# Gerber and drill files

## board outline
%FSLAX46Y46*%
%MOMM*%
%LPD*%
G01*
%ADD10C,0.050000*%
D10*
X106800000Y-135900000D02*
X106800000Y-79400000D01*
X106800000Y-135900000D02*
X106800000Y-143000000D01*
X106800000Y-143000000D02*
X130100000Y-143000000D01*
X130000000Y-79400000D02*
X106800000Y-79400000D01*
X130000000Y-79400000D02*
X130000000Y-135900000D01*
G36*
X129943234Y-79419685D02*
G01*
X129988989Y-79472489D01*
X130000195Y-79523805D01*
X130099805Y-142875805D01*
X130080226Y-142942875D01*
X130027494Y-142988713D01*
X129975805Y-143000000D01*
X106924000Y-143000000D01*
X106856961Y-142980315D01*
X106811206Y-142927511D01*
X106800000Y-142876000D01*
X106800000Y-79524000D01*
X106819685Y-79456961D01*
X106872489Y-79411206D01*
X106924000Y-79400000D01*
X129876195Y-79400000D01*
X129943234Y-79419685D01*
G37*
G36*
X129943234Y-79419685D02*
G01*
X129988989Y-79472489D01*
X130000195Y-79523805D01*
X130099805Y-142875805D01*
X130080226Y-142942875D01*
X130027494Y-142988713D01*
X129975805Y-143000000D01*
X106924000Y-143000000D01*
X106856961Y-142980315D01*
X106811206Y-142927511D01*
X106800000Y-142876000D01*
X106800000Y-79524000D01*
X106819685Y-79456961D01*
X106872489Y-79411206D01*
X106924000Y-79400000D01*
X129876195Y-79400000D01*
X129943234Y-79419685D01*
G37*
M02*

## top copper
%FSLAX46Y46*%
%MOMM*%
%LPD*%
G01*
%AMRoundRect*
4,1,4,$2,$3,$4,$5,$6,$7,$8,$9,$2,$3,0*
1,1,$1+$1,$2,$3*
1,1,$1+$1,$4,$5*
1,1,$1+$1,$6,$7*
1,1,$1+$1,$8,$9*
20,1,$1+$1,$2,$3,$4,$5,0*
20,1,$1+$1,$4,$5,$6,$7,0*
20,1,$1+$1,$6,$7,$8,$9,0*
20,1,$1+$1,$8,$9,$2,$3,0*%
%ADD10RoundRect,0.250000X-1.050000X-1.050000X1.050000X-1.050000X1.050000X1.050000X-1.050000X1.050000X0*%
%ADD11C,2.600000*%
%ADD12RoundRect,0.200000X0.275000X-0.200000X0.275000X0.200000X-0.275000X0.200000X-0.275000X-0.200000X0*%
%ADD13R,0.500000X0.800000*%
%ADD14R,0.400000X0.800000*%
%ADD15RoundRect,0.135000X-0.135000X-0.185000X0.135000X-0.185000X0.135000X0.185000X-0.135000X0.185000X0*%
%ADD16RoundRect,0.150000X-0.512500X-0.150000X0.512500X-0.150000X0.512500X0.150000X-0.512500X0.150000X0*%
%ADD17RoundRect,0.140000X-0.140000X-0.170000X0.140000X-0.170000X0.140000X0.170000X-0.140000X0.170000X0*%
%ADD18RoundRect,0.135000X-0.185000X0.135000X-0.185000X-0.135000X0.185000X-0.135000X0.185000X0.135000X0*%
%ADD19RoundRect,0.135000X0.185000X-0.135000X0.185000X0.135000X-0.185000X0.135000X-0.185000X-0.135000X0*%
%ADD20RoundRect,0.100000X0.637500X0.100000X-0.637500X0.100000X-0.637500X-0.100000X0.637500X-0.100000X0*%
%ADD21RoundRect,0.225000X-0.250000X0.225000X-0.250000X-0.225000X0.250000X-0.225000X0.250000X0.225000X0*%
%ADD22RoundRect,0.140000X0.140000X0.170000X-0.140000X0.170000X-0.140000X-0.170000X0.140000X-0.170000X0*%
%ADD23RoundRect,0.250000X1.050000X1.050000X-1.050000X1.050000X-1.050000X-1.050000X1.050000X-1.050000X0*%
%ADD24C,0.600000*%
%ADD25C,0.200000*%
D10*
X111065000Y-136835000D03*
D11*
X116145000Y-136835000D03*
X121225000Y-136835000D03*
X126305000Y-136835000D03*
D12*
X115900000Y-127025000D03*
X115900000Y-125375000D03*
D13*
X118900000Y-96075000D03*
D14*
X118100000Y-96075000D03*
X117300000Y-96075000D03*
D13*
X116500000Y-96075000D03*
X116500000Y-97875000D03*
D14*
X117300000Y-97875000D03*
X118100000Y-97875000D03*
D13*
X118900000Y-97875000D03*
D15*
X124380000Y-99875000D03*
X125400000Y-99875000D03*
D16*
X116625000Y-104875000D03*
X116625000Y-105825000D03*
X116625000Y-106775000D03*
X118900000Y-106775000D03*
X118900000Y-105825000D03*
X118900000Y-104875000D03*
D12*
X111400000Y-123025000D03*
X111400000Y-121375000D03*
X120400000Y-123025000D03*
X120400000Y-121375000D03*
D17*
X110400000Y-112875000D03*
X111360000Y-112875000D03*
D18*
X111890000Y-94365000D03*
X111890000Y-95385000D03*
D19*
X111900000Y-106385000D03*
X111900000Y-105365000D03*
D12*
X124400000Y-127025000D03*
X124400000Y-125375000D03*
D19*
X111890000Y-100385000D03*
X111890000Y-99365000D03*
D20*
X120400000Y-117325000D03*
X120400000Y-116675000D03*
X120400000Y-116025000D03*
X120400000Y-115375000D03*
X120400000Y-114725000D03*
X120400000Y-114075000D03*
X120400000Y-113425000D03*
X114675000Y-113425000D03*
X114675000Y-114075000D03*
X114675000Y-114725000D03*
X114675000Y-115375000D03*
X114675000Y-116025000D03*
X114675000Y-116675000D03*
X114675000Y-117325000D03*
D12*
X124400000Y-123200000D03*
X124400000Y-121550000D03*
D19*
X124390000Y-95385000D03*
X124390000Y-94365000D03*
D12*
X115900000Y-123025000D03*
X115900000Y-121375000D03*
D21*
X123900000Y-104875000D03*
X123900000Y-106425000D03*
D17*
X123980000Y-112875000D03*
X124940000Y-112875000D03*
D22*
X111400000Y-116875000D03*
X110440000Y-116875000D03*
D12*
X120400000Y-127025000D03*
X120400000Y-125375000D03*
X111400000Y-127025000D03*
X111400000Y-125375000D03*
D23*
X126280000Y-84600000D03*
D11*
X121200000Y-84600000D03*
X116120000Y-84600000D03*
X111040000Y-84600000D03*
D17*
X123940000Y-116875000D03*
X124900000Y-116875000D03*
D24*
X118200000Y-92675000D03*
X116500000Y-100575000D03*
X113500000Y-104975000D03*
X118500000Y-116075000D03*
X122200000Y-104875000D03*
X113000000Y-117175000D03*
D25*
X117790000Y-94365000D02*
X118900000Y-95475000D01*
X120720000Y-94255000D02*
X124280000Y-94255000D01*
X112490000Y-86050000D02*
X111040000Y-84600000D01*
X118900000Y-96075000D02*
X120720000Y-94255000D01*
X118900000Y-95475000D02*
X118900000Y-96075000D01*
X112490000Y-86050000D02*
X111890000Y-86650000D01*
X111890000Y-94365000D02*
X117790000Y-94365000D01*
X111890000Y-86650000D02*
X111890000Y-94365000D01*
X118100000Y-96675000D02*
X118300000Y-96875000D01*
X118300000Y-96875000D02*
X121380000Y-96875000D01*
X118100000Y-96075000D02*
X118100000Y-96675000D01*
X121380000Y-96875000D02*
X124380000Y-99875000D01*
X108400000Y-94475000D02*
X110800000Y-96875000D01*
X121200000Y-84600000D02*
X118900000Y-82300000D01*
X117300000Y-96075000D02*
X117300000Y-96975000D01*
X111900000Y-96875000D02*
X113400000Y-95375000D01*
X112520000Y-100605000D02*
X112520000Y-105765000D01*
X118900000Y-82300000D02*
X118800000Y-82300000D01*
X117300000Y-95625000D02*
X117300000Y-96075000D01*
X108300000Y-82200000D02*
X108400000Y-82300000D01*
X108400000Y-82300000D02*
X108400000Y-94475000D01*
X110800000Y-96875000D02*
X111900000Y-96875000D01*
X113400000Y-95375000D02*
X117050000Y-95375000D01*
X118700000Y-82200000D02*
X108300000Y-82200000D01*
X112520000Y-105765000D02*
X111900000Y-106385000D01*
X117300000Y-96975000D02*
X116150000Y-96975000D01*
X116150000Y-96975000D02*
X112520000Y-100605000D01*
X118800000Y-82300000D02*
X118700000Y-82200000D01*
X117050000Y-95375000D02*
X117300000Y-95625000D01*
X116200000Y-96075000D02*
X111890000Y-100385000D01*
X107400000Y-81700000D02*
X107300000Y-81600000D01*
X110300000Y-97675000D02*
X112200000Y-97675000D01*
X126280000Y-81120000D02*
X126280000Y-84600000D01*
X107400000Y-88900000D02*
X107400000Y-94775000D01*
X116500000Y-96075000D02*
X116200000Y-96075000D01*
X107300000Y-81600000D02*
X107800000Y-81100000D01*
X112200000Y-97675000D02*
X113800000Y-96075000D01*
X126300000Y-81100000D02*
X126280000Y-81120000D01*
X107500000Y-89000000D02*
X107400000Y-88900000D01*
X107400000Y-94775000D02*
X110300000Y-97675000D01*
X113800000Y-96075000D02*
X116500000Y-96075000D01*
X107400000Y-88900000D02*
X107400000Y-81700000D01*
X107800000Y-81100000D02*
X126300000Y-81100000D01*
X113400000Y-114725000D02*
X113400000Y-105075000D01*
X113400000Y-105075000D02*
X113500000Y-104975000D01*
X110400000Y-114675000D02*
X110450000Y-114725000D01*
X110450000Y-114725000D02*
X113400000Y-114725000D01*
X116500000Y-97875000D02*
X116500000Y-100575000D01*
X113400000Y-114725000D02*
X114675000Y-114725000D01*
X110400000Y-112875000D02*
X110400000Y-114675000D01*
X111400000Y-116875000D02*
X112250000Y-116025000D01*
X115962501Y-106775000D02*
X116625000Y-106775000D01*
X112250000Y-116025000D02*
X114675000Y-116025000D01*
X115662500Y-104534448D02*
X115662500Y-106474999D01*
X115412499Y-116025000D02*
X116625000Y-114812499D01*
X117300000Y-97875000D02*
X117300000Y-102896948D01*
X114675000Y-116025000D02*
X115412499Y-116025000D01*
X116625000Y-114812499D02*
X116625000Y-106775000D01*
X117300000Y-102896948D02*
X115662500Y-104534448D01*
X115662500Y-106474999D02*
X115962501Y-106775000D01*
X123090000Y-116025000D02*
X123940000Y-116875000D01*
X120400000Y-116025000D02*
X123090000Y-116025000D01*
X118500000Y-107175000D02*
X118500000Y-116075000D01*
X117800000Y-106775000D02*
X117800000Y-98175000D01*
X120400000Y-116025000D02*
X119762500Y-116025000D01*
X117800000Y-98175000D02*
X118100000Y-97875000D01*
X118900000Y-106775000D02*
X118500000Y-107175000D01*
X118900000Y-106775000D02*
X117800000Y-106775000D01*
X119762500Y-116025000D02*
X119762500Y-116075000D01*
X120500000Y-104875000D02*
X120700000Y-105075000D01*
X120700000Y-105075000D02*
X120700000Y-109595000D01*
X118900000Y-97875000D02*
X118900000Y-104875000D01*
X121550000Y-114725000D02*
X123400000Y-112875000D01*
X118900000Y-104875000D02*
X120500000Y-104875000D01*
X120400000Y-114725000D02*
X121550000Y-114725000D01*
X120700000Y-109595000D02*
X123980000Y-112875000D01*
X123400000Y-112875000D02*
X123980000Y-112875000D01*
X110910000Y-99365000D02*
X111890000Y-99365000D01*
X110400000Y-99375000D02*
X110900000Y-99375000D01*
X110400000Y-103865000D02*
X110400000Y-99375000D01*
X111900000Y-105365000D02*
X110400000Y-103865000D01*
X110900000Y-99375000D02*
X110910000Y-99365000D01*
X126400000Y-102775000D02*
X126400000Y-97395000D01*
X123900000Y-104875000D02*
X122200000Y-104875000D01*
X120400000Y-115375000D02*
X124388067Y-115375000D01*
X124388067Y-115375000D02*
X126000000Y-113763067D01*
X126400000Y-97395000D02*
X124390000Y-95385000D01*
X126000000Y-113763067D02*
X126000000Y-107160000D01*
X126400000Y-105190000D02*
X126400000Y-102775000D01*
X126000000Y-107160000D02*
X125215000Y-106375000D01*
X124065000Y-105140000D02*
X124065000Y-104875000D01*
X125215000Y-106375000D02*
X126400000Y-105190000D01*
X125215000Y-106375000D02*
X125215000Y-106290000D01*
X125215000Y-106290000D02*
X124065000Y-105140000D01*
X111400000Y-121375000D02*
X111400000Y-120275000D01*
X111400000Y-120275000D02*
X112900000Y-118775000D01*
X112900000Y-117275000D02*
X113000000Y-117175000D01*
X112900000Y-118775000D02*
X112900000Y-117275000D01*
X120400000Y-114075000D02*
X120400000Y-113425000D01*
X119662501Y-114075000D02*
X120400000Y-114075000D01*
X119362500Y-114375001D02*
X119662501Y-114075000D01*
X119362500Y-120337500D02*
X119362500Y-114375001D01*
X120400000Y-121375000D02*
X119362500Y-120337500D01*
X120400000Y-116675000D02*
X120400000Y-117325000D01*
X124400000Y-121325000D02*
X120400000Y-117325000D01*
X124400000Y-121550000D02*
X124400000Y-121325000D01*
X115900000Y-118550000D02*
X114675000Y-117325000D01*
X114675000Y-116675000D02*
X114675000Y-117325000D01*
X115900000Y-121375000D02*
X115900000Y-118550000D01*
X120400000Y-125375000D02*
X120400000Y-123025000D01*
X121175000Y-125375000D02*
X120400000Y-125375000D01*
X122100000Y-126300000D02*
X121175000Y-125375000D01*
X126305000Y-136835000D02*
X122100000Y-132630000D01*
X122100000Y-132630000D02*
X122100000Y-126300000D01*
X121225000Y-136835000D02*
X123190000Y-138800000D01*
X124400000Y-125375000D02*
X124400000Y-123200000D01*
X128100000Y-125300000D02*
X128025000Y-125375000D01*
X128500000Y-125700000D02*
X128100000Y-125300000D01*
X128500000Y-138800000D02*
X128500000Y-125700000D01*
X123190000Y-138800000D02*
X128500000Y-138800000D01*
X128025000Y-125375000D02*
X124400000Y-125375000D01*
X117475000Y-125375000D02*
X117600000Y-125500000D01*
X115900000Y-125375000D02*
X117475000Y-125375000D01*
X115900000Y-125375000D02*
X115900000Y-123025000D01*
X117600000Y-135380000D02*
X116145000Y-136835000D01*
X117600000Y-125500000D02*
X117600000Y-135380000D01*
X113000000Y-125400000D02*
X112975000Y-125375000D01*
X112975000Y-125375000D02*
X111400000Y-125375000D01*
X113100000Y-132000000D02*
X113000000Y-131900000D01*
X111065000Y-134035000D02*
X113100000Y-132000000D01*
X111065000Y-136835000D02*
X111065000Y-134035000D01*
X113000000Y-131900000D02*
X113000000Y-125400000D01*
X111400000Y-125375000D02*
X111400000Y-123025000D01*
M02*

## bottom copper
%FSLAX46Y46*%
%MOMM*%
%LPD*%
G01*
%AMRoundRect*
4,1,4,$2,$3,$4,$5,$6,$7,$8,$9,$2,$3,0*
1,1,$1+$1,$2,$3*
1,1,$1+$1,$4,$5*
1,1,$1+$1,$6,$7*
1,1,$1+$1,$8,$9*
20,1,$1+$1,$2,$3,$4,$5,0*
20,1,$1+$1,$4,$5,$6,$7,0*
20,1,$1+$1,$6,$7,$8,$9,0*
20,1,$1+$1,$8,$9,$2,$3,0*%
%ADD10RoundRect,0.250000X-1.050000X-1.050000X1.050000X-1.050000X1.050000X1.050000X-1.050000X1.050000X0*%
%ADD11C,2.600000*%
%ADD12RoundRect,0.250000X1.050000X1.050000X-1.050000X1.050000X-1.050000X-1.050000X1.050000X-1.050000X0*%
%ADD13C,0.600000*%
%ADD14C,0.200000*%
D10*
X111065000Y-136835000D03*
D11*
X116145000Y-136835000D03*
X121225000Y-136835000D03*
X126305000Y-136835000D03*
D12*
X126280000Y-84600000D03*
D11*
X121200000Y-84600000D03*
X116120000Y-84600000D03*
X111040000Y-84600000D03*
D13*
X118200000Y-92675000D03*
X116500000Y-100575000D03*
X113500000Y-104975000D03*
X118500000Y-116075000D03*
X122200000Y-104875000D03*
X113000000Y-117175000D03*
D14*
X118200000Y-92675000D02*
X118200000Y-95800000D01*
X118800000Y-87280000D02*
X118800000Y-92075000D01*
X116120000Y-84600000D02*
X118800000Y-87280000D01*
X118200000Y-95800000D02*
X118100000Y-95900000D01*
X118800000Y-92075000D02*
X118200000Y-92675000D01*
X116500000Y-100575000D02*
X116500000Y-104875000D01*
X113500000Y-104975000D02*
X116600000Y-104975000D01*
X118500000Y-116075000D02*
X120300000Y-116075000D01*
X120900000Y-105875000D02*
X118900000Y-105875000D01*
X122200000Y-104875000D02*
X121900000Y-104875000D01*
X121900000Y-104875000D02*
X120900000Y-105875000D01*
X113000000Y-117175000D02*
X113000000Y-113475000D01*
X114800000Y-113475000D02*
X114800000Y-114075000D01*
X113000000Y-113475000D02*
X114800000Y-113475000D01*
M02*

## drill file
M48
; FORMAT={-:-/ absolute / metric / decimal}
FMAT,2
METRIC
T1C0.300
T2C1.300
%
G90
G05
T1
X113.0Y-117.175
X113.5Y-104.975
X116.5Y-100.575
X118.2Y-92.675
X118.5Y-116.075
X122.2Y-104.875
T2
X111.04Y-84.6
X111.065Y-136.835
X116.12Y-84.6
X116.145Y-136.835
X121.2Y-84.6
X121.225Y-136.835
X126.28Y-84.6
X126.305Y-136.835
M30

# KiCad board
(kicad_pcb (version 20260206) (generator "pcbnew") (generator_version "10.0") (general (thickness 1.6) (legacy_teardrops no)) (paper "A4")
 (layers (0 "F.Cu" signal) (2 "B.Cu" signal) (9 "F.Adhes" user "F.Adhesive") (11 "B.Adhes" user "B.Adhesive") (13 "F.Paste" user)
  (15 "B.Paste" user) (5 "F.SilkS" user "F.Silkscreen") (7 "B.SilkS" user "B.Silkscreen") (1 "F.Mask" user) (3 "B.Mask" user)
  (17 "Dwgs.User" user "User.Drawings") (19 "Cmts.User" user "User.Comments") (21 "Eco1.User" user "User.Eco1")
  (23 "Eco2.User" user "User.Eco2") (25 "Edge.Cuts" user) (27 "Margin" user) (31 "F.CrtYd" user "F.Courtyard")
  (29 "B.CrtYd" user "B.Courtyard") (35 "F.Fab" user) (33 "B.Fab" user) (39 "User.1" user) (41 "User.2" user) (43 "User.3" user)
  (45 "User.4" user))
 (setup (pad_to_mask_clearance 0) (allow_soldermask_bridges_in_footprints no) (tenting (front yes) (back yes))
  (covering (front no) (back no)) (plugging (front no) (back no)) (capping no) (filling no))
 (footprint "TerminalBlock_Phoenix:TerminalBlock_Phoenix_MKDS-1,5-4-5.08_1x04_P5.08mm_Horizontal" (layer "F.Cu") (at 111.065 136.835)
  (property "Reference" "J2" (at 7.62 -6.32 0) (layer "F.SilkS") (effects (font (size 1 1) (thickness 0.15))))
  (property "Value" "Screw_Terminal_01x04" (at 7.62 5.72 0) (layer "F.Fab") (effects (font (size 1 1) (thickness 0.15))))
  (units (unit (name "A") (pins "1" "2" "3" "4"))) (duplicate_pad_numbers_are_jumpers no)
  (pad "1" thru_hole roundrect (at 0 0) (size 2.6 2.6) (drill 1.3) (layers "*.Cu" "*.Mask") (remove_unused_layers no)
   (roundrect_rratio 0.096154) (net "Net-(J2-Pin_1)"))
  (pad "2" thru_hole circle (at 5.08 0) (size 2.6 2.6) (drill 1.3) (layers "*.Cu" "*.Mask") (remove_unused_layers no) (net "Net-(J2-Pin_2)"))
  (pad "3" thru_hole circle (at 10.16 0) (size 2.6 2.6) (drill 1.3) (layers "*.Cu" "*.Mask") (remove_unused_layers no)
   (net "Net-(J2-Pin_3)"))
  (pad "4" thru_hole circle (at 15.24 0) (size 2.6 2.6) (drill 1.3) (layers "*.Cu" "*.Mask") (remove_unused_layers no)
   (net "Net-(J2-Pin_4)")))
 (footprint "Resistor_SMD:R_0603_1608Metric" (layer "F.Cu") (at 115.9 126.2 90)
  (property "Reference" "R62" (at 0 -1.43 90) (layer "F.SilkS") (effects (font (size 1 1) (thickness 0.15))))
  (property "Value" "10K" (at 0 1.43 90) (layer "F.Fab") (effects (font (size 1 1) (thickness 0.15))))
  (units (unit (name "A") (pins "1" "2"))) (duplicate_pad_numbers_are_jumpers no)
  (pad "1" smd roundrect (at -0.825 0 90) (size 0.8 0.95) (layers "F.Cu" "F.Mask" "F.Paste") (roundrect_rratio 0.25) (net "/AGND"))
  (pad "2" smd roundrect (at 0.825 0 90) (size 0.8 0.95) (layers "F.Cu" "F.Mask" "F.Paste") (roundrect_rratio 0.25) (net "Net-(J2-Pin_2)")))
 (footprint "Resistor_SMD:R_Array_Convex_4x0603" (layer "F.Cu") (at 117.7 96.975 -90)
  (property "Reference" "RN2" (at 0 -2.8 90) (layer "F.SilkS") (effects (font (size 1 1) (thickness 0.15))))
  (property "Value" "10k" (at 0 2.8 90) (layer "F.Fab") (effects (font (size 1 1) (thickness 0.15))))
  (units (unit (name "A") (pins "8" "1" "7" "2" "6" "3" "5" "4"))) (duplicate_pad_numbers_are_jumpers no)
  (pad "1" smd rect (at -0.9 -1.2 270) (size 0.8 0.5) (layers "F.Cu" "F.Mask" "F.Paste") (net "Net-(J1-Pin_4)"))
  (pad "2" smd rect (at -0.9 -0.4 270) (size 0.8 0.4) (layers "F.Cu" "F.Mask" "F.Paste") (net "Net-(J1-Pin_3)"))
  (pad "3" smd rect (at -0.9 0.4 270) (size 0.8 0.4) (layers "F.Cu" "F.Mask" "F.Paste") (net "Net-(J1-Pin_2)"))
  (pad "4" smd rect (at -0.9 1.2 270) (size 0.8 0.5) (layers "F.Cu" "F.Mask" "F.Paste") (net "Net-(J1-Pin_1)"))
  (pad "5" smd rect (at 0.9 1.2 270) (size 0.8 0.5) (layers "F.Cu" "F.Mask" "F.Paste") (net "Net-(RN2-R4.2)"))
  (pad "6" smd rect (at 0.9 0.4 270) (size 0.8 0.4) (layers "F.Cu" "F.Mask" "F.Paste") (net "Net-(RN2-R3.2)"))
  (pad "7" smd rect (at 0.9 -0.4 270) (size 0.8 0.4) (layers "F.Cu" "B.Mask" "F.Paste") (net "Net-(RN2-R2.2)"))
  (pad "8" smd rect (at 0.9 -1.2 270) (size 0.8 0.5) (layers "F.Cu" "F.Mask" "F.Paste") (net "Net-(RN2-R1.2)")))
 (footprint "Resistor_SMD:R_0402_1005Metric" (layer "F.Cu") (at 124.89 99.875)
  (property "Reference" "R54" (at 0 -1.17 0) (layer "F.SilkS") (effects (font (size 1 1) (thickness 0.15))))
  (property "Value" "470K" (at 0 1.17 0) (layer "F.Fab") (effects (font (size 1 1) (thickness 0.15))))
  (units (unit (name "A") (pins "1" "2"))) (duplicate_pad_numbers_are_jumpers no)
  (pad "1" smd roundrect (at -0.51 0) (size 0.54 0.64) (layers "F.Cu" "F.Mask" "F.Paste") (roundrect_rratio 0.25) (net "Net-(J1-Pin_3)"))
  (pad "2" smd roundrect (at 0.51 0) (size 0.54 0.64) (layers "F.Cu" "F.Mask" "F.Paste") (roundrect_rratio 0.25) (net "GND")))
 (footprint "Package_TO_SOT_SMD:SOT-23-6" (layer "F.Cu") (at 117.7625 105.825)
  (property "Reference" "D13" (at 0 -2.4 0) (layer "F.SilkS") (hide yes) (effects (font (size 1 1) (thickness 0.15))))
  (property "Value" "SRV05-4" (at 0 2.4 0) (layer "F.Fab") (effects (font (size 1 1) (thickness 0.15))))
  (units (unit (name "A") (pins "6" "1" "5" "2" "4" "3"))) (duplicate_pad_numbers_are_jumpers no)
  (pad "1" smd roundrect (at -1.1375 -0.95) (size 1.325 0.6) (layers "F.Cu" "F.Mask" "F.Paste") (roundrect_rratio 0.25)
   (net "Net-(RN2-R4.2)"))
  (pad "2" smd roundrect (at -1.1375 0) (size 1.325 0.6) (layers "F.Cu" "F.Mask" "F.Paste") (roundrect_rratio 0.25) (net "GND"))
  (pad "3" smd roundrect (at -1.1375 0.95) (size 1.325 0.6) (layers "F.Cu" "F.Mask" "F.Paste") (roundrect_rratio 0.25)
   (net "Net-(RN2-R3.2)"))
  (pad "4" smd roundrect (at 1.1375 0.95) (size 1.325 0.6) (layers "F.Cu" "F.Mask" "F.Paste") (roundrect_rratio 0.25) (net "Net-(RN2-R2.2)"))
  (pad "5" smd roundrect (at 1.1375 0) (size 1.325 0.6) (layers "F.Cu" "F.Mask" "F.Paste") (roundrect_rratio 0.25) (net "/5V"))
  (pad "6" smd roundrect (at 1.1375 -0.95) (size 1.325 0.6) (layers "F.Cu" "F.Mask" "F.Paste") (roundrect_rratio 0.25)
   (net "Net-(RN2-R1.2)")))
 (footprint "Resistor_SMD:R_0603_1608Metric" (layer "F.Cu") (at 111.4 122.2 90)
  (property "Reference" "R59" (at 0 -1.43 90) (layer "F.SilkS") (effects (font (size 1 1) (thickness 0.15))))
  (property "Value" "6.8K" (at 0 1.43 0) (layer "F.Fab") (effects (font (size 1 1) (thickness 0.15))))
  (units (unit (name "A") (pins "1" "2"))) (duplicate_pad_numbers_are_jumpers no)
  (pad "1" smd roundrect (at -0.825 0 90) (size 0.8 0.95) (layers "F.Cu" "F.Mask" "F.Paste") (roundrect_rratio 0.25) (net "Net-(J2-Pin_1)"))
  (pad "2" smd roundrect (at 0.825 0 90) (size 0.8 0.95) (layers "F.Cu" "F.Mask" "F.Paste") (roundrect_rratio 0.25) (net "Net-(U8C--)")))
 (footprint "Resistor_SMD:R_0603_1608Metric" (layer "F.Cu") (at 120.4 122.2 90)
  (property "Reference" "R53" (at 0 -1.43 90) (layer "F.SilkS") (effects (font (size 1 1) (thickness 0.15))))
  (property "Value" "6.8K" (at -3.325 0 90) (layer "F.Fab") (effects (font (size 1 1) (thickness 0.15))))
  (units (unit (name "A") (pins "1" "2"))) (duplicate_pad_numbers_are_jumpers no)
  (pad "1" smd roundrect (at -0.825 0 90) (size 0.8 0.95) (layers "F.Cu" "F.Mask" "F.Paste") (roundrect_rratio 0.25) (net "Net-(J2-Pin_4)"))
  (pad "2" smd roundrect (at 0.825 0 90) (size 0.8 0.95) (layers "F.Cu" "F.Mask" "F.Paste") (roundrect_rratio 0.25) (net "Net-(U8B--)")))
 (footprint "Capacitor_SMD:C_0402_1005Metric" (layer "F.Cu") (at 110.88 112.875)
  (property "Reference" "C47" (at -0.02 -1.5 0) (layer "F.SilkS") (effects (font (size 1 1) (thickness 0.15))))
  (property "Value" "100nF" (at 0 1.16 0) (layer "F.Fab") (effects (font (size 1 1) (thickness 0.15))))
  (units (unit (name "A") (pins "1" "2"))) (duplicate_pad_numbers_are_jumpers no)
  (pad "1" smd roundrect (at -0.48 0) (size 0.56 0.62) (layers "F.Cu" "F.Mask" "F.Paste") (roundrect_rratio 0.25) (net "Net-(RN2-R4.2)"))
  (pad "2" smd roundrect (at 0.48 0) (size 0.56 0.62) (layers "F.Cu" "F.Mask" "F.Paste") (roundrect_rratio 0.25) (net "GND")))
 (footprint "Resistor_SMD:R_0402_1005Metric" (layer "F.Cu") (at 111.89 94.875 -90)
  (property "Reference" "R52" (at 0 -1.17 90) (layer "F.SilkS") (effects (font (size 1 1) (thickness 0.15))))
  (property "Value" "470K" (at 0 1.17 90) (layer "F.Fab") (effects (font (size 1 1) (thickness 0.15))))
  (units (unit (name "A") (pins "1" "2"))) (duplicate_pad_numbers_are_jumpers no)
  (pad "1" smd roundrect (at -0.51 0 270) (size 0.54 0.64) (layers "F.Cu" "F.Mask" "F.Paste") (roundrect_rratio 0.25) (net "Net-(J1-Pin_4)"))
  (pad "2" smd roundrect (at 0.51 0 270) (size 0.54 0.64) (layers "F.Cu" "F.Mask" "F.Paste") (roundrect_rratio 0.25) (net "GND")))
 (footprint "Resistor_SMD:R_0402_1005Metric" (layer "F.Cu") (at 111.9 105.875 90)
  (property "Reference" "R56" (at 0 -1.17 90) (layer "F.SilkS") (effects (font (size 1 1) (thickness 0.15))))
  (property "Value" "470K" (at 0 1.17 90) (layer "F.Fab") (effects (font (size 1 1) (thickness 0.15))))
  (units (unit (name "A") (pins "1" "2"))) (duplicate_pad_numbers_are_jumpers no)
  (pad "1" smd roundrect (at -0.51 0 90) (size 0.54 0.64) (layers "F.Cu" "F.Mask" "F.Paste") (roundrect_rratio 0.25) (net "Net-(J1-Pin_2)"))
  (pad "2" smd roundrect (at 0.51 0 90) (size 0.54 0.64) (layers "F.Cu" "F.Mask" "F.Paste") (roundrect_rratio 0.25) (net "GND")))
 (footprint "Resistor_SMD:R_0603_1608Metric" (layer "F.Cu") (at 124.4 126.2 90)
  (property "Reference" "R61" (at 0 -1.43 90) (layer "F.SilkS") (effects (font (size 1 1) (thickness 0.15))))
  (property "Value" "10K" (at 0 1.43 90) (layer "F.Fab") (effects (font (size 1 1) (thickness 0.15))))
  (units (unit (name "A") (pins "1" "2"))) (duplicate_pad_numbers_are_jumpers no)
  (pad "1" smd roundrect (at -0.825 0 90) (size 0.8 0.95) (layers "F.Cu" "F.Mask" "F.Paste") (roundrect_rratio 0.25) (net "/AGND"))
  (pad "2" smd roundrect (at 0.825 0 90) (size 0.8 0.95) (layers "F.Cu" "F.Mask" "F.Paste") (roundrect_rratio 0.25) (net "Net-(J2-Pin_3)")))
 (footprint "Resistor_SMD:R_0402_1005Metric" (layer "F.Cu") (at 111.89 99.875 90)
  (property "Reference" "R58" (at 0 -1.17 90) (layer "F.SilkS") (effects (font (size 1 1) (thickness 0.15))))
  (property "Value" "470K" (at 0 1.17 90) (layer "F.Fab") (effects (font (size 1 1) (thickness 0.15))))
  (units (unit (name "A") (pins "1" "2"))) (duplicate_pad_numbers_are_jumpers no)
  (pad "1" smd roundrect (at -0.51 0 90) (size 0.54 0.64) (layers "F.Cu" "F.Mask" "F.Paste") (roundrect_rratio 0.25) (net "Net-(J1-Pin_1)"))
  (pad "2" smd roundrect (at 0.51 0 90) (size 0.54 0.64) (layers "F.Cu" "F.Mask" "F.Paste") (roundrect_rratio 0.25) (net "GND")))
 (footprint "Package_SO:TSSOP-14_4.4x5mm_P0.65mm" (layer "F.Cu") (at 117.5375 115.375 180)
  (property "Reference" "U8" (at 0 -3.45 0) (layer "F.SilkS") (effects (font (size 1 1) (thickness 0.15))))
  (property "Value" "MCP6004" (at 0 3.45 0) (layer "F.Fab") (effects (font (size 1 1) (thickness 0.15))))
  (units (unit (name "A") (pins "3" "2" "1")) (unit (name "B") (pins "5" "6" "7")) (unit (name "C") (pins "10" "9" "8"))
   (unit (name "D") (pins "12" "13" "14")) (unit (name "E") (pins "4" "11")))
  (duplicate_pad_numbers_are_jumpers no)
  (pad "1" smd roundrect (at -2.8625 -1.95 180) (size 1.475 0.4) (layers "F.Cu" "F.Mask" "F.Paste") (roundrect_rratio 0.25)
   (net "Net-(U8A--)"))
  (pad "2" smd roundrect (at -2.8625 -1.3 180) (size 1.475 0.4) (layers "F.Cu" "F.Mask" "F.Paste") (roundrect_rratio 0.25)
   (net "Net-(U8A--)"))
  (pad "3" smd roundrect (at -2.8625 -0.65 180) (size 1.475 0.4) (layers "F.Cu" "F.Mask" "F.Paste") (roundrect_rratio 0.25)
   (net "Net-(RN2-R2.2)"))
  (pad "4" smd roundrect (at -2.8625 0 180) (size 1.475 0.4) (layers "F.Cu" "F.Mask" "F.Paste") (roundrect_rratio 0.25) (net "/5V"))
  (pad "5" smd roundrect (at -2.8625 0.65 180) (size 1.475 0.4) (layers "F.Cu" "F.Mask" "F.Paste") (roundrect_rratio 0.25)
   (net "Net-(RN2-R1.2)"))
  (pad "6" smd roundrect (at -2.8625 1.3 180) (size 1.475 0.4) (layers "F.Cu" "F.Mask" "F.Paste") (roundrect_rratio 0.25)
   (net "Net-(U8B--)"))
  (pad "7" smd roundrect (at -2.8625 1.95 180) (size 1.475 0.4) (layers "F.Cu" "F.Mask" "F.Paste") (roundrect_rratio 0.25)
   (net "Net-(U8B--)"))
  (pad "8" smd roundrect (at 2.8625 1.95 180) (size 1.475 0.4) (layers "F.Cu" "F.Mask" "F.Paste") (roundrect_rratio 0.25)
   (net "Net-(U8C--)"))
  (pad "9" smd roundrect (at 2.8625 1.3 180) (size 1.475 0.4) (layers "F.Cu" "F.Mask" "F.Paste") (roundrect_rratio 0.25) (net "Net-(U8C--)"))
  (pad "10" smd roundrect (at 2.8625 0.65 180) (size 1.475 0.4) (layers "F.Cu" "F.Mask" "F.Paste") (roundrect_rratio 0.25)
   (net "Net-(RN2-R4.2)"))
  (pad "11" smd roundrect (at 2.8625 0 180) (size 1.475 0.4) (layers "F.Cu" "F.Mask" "F.Paste") (roundrect_rratio 0.25)
   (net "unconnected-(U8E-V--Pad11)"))
  (pad "12" smd roundrect (at 2.8625 -0.65 180) (size 1.475 0.4) (layers "F.Cu" "F.Mask" "F.Paste") (roundrect_rratio 0.25)
   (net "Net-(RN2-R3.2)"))
  (pad "13" smd roundrect (at 2.8625 -1.3 180) (size 1.475 0.4) (layers "F.Cu" "F.Mask" "F.Paste") (roundrect_rratio 0.25)
   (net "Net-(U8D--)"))
  (pad "14" smd roundrect (at 2.8625 -1.95 180) (size 1.475 0.4) (layers "F.Cu" "F.Mask" "F.Paste") (roundrect_rratio 0.25)
   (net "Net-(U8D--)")))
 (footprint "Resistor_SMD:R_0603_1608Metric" (layer "F.Cu") (at 124.4 122.375 90)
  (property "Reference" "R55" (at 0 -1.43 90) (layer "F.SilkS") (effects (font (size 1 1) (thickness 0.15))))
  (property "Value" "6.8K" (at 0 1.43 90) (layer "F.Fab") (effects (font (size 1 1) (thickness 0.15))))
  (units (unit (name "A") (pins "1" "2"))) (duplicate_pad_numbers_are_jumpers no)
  (pad "1" smd roundrect (at -0.825 0 90) (size 0.8 0.95) (layers "F.Cu" "F.Mask" "F.Paste") (roundrect_rratio 0.25) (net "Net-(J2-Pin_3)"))
  (pad "2" smd roundrect (at 0.825 0 90) (size 0.8 0.95) (layers "F.Cu" "F.Mask" "F.Paste") (roundrect_rratio 0.25) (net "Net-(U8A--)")))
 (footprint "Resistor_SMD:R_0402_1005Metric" (layer "F.Cu") (at 124.39 94.875 90)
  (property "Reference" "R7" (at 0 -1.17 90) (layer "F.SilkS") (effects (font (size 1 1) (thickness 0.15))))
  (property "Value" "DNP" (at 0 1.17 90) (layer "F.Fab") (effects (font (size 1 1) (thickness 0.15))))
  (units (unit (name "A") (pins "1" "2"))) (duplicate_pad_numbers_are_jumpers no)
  (pad "1" smd roundrect (at -0.51 0 90) (size 0.54 0.64) (layers "F.Cu" "F.Mask" "F.Paste") (roundrect_rratio 0.25) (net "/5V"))
  (pad "2" smd roundrect (at 0.51 0 90) (size 0.54 0.64) (layers "F.Cu" "F.Mask" "F.Paste") (roundrect_rratio 0.25) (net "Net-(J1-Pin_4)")))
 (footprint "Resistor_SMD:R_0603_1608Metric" (layer "F.Cu") (at 115.9 122.2 90)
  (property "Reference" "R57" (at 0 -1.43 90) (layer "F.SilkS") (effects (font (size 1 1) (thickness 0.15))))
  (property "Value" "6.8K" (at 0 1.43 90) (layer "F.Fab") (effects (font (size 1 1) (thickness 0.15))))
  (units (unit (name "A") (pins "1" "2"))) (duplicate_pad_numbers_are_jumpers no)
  (pad "1" smd roundrect (at -0.825 0 90) (size 0.8 0.95) (layers "F.Cu" "F.Mask" "F.Paste") (roundrect_rratio 0.25) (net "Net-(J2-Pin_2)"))
  (pad "2" smd roundrect (at 0.825 0 90) (size 0.8 0.95) (layers "F.Cu" "F.Mask" "F.Paste") (roundrect_rratio 0.25) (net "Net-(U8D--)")))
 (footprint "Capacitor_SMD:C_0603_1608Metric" (layer "F.Cu") (at 123.9 105.65 -90)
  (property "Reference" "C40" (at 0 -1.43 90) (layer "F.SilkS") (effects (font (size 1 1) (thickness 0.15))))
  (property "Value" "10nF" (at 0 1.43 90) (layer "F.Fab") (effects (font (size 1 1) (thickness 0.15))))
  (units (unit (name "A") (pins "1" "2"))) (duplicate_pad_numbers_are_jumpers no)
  (pad "1" smd roundrect (at -0.775 0 270) (size 0.9 0.95) (layers "F.Cu" "F.Mask" "F.Paste") (roundrect_rratio 0.25) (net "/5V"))
  (pad "2" smd roundrect (at 0.775 0 270) (size 0.9 0.95) (layers "F.Cu" "F.Mask" "F.Paste") (roundrect_rratio 0.25) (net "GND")))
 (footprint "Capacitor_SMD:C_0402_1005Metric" (layer "F.Cu") (at 124.46 112.875)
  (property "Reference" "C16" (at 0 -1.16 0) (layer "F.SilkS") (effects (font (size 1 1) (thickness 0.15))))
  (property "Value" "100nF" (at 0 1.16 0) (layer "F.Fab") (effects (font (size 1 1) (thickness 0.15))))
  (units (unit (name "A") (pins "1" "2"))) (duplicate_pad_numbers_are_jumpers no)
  (pad "1" smd roundrect (at -0.48 0) (size 0.56 0.62) (layers "F.Cu" "F.Mask" "F.Paste") (roundrect_rratio 0.25) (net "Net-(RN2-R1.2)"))
  (pad "2" smd roundrect (at 0.48 0) (size 0.56 0.62) (layers "F.Cu" "F.Mask" "F.Paste") (roundrect_rratio 0.25) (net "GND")))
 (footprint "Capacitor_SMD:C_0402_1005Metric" (layer "F.Cu") (at 110.92 116.875 180)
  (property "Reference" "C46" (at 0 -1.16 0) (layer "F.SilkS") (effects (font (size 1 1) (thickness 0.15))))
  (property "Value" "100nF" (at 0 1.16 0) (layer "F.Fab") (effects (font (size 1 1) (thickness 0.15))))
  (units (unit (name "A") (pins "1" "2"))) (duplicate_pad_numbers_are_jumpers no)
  (pad "1" smd roundrect (at -0.48 0 180) (size 0.56 0.62) (layers "F.Cu" "F.Mask" "F.Paste") (roundrect_rratio 0.25) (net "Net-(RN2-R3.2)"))
  (pad "2" smd roundrect (at 0.48 0 180) (size 0.56 0.62) (layers "F.Cu" "F.Mask" "F.Paste") (roundrect_rratio 0.25) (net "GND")))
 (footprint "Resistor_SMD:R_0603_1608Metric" (layer "F.Cu") (at 120.4 126.2 90)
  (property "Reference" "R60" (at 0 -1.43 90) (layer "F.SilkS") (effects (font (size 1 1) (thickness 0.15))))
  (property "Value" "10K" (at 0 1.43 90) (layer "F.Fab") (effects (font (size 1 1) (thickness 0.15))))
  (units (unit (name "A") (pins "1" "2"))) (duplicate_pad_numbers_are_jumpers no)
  (pad "1" smd roundrect (at -0.825 0 90) (size 0.8 0.95) (layers "F.Cu" "F.Mask" "F.Paste") (roundrect_rratio 0.25) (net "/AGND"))
  (pad "2" smd roundrect (at 0.825 0 90) (size 0.8 0.95) (layers "F.Cu" "F.Mask" "F.Paste") (roundrect_rratio 0.25) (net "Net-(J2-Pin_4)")))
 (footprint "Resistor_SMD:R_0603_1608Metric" (layer "F.Cu") (at 111.4 126.2 90)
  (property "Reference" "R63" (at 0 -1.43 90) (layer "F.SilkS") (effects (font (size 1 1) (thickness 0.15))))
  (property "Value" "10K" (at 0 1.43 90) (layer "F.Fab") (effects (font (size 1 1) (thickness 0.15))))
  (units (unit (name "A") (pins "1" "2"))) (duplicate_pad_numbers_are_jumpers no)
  (pad "1" smd roundrect (at -0.825 0 90) (size 0.8 0.95) (layers "F.Cu" "F.Mask" "F.Paste") (roundrect_rratio 0.25) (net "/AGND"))
  (pad "2" smd roundrect (at 0.825 0 90) (size 0.8 0.95) (layers "F.Cu" "F.Mask" "F.Paste") (roundrect_rratio 0.25) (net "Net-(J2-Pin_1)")))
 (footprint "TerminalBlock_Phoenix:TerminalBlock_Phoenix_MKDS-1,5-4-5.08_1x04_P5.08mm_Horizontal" (layer "F.Cu") (at 126.28 84.6 180)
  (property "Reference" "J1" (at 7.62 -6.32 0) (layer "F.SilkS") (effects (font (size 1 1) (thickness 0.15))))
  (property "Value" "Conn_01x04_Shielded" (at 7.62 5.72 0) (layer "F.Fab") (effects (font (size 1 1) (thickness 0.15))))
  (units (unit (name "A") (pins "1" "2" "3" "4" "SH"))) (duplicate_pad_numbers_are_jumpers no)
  (pad "1" thru_hole roundrect (at 0 0 180) (size 2.6 2.6) (drill 1.3) (layers "*.Cu" "*.Mask") (remove_unused_layers no)
   (roundrect_rratio 0.096154) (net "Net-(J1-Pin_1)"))
  (pad "2" thru_hole circle (at 5.08 0 180) (size 2.6 2.6) (drill 1.3) (layers "*.Cu" "*.Mask") (remove_unused_layers no)
   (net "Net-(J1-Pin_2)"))
  (pad "3" thru_hole circle (at 10.16 0 180) (size 2.6 2.6) (drill 1.3) (layers "*.Cu" "*.Mask") (remove_unused_layers no)
   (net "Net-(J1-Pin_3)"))
  (pad "4" thru_hole circle (at 15.24 0 180) (size 2.6 2.6) (drill 1.3) (layers "*.Cu" "*.Mask") (remove_unused_layers no)
   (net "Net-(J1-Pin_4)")))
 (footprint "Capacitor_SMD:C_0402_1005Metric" (layer "F.Cu") (at 124.42 116.875)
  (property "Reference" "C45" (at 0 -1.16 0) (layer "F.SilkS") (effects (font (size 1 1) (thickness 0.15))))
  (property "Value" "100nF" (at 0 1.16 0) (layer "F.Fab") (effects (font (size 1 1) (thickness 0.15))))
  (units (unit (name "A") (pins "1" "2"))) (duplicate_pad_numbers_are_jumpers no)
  (pad "1" smd roundrect (at -0.48 0) (size 0.56 0.62) (layers "F.Cu" "F.Mask" "F.Paste") (roundrect_rratio 0.25) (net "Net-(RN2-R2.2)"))
  (pad "2" smd roundrect (at 0.48 0) (size 0.56 0.62) (layers "F.Cu" "F.Mask" "F.Paste") (roundrect_rratio 0.25) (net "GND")))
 (gr_line (start 106.8 135.9) (end 106.8 79.4) (stroke (width 0.05) (type default)) (layer "Edge.Cuts"))
 (gr_line (start 106.8 135.9) (end 106.8 143) (stroke (width 0.05) (type default)) (layer "Edge.Cuts"))
 (gr_line (start 106.8 143) (end 130.1 143) (stroke (width 0.05) (type default)) (layer "Edge.Cuts"))
 (gr_line (start 130 79.4) (end 106.8 79.4) (stroke (width 0.05) (type default)) (layer "Edge.Cuts"))
 (gr_line (start 130 79.4) (end 130 135.9) (stroke (width 0.05) (type default)) (layer "Edge.Cuts"))
 (segment (start 117.79 94.365) (end 118.9 95.475) (width 0.2) (layer "F.Cu") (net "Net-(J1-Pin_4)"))
 (segment (start 120.72 94.255) (end 124.28 94.255) (width 0.2) (layer "F.Cu") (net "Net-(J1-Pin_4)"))
 (segment (start 112.49 86.05) (end 111.04 84.6) (width 0.2) (layer "F.Cu") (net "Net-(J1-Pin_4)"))
 (segment (start 118.9 96.075) (end 120.72 94.255) (width 0.2) (layer "F.Cu") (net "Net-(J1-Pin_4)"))
 (segment (start 118.9 95.475) (end 118.9 96.075) (width 0.2) (layer "F.Cu") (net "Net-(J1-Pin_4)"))
 (segment (start 112.49 86.05) (end 111.89 86.65) (width 0.2) (layer "F.Cu") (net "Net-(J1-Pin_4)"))
 (segment (start 111.89 94.365) (end 117.79 94.365) (width 0.2) (layer "F.Cu") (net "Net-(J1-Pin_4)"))
 (segment (start 111.89 86.65) (end 111.89 94.365) (width 0.2) (layer "F.Cu") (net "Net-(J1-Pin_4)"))
 (segment (start 118.1 96.675) (end 118.3 96.875) (width 0.2) (layer "F.Cu") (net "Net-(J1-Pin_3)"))
 (segment (start 118.3 96.875) (end 121.38 96.875) (width 0.2) (layer "F.Cu") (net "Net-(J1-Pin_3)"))
 (segment (start 118.1 96.075) (end 118.1 96.675) (width 0.2) (layer "F.Cu") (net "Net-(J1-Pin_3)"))
 (segment (start 121.38 96.875) (end 124.38 99.875) (width 0.2) (layer "F.Cu") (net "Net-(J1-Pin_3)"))
 (via (at 118.2 92.675) (size 0.6) (drill 0.3) (layers "F.Cu" "B.Cu") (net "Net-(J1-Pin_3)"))
 (segment (start 118.2 92.675) (end 118.2 95.8) (width 0.2) (layer "B.Cu") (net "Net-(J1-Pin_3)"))
 (segment (start 118.8 87.28) (end 118.8 92.075) (width 0.2) (layer "B.Cu") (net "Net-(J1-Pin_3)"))
 (segment (start 116.12 84.6) (end 118.8 87.28) (width 0.2) (layer "B.Cu") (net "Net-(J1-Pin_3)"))
 (segment (start 118.2 95.8) (end 118.1 95.9) (width 0.2) (layer "B.Cu") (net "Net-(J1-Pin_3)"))
 (segment (start 118.8 92.075) (end 118.2 92.675) (width 0.2) (layer "B.Cu") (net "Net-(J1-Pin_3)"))
 (segment (start 108.4 94.475) (end 110.8 96.875) (width 0.2) (layer "F.Cu") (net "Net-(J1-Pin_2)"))
 (segment (start 121.2 84.6) (end 118.9 82.3) (width 0.2) (layer "F.Cu") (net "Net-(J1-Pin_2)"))
 (segment (start 117.3 96.075) (end 117.3 96.975) (width 0.2) (layer "F.Cu") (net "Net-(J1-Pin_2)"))
 (segment (start 111.9 96.875) (end 113.4 95.375) (width 0.2) (layer "F.Cu") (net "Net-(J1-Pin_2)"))
 (segment (start 112.52 100.605) (end 112.52 105.765) (width 0.2) (layer "F.Cu") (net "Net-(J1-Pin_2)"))
 (segment (start 118.9 82.3) (end 118.8 82.3) (width 0.2) (layer "F.Cu") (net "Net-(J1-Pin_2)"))
 (segment (start 117.3 95.625) (end 117.3 96.075) (width 0.2) (layer "F.Cu") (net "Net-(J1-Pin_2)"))
 (segment (start 108.3 82.2) (end 108.4 82.3) (width 0.2) (layer "F.Cu") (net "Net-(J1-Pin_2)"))
 (segment (start 108.4 82.3) (end 108.4 94.475) (width 0.2) (layer "F.Cu") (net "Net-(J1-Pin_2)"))
 (segment (start 110.8 96.875) (end 111.9 96.875) (width 0.2) (layer "F.Cu") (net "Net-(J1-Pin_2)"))
 (segment (start 113.4 95.375) (end 117.05 95.375) (width 0.2) (layer "F.Cu") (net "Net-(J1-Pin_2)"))
 (segment (start 118.7 82.2) (end 108.3 82.2) (width 0.2) (layer "F.Cu") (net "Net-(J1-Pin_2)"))
 (segment (start 112.52 105.765) (end 111.9 106.385) (width 0.2) (layer "F.Cu") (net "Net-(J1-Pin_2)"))
 (segment (start 117.3 96.975) (end 116.15 96.975) (width 0.2) (layer "F.Cu") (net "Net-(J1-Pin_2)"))
 (segment (start 116.15 96.975) (end 112.52 100.605) (width 0.2) (layer "F.Cu") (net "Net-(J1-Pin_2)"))
 (segment (start 118.8 82.3) (end 118.7 82.2) (width 0.2) (layer "F.Cu") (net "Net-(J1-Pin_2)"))
 (segment (start 117.05 95.375) (end 117.3 95.625) (width 0.2) (layer "F.Cu") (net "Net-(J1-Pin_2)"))
 (segment (start 116.2 96.075) (end 111.89 100.385) (width 0.2) (layer "F.Cu") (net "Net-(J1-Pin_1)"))
 (segment (start 107.4 81.7) (end 107.3 81.6) (width 0.2) (layer "F.Cu") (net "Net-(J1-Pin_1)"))
 (segment (start 110.3 97.675) (end 112.2 97.675) (width 0.2) (layer "F.Cu") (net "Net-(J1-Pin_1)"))
 (segment (start 126.28 81.12) (end 126.28 84.6) (width 0.2) (layer "F.Cu") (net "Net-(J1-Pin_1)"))
 (segment (start 107.4 88.9) (end 107.4 94.775) (width 0.2) (layer "F.Cu") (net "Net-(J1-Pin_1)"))
 (segment (start 116.5 96.075) (end 116.2 96.075) (width 0.2) (layer "F.Cu") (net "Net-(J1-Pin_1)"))
 (segment (start 107.3 81.6) (end 107.8 81.1) (width 0.2) (layer "F.Cu") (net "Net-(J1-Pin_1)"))
 (segment (start 112.2 97.675) (end 113.8 96.075) (width 0.2) (layer "F.Cu") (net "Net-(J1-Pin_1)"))
 (segment (start 126.3 81.1) (end 126.28 81.12) (width 0.2) (layer "F.Cu") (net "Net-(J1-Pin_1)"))
 (segment (start 107.5 89) (end 107.4 88.9) (width 0.2) (layer "F.Cu") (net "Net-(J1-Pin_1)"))
 (segment (start 107.4 94.775) (end 110.3 97.675) (width 0.2) (layer "F.Cu") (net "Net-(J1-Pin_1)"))
 (segment (start 113.8 96.075) (end 116.5 96.075) (width 0.2) (layer "F.Cu") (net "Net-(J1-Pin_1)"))
 (segment (start 107.4 88.9) (end 107.4 81.7) (width 0.2) (layer "F.Cu") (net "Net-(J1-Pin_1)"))
 (segment (start 107.8 81.1) (end 126.3 81.1) (width 0.2) (layer "F.Cu") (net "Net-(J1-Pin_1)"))
 (segment (start 113.4 114.725) (end 113.4 105.075) (width 0.2) (layer "F.Cu") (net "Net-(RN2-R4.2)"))
 (segment (start 113.4 105.075) (end 113.5 104.975) (width 0.2) (layer "F.Cu") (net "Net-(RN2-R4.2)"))
 (segment (start 110.4 114.675) (end 110.45 114.725) (width 0.2) (layer "F.Cu") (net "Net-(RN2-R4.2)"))
 (segment (start 110.45 114.725) (end 113.4 114.725) (width 0.2) (layer "F.Cu") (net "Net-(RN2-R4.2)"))
 (segment (start 116.5 97.875) (end 116.5 100.575) (width 0.2) (layer "F.Cu") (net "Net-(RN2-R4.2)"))
 (segment (start 113.4 114.725) (end 114.675 114.725) (width 0.2) (layer "F.Cu") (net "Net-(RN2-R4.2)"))
 (segment (start 110.4 112.875) (end 110.4 114.675) (width 0.2) (layer "F.Cu") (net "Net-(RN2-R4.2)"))
 (via (at 116.5 100.575) (size 0.6) (drill 0.3) (layers "F.Cu" "B.Cu") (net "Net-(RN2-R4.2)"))
 (via (at 113.5 104.975) (size 0.6) (drill 0.3) (layers "F.Cu" "B.Cu") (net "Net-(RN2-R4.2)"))
 (segment (start 116.5 100.575) (end 116.5 104.875) (width 0.2) (layer "B.Cu") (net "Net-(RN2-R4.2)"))
 (segment (start 113.5 104.975) (end 116.6 104.975) (width 0.2) (layer "B.Cu") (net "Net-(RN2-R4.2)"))
 (segment (start 111.4 116.875) (end 112.25 116.025) (width 0.2) (layer "F.Cu") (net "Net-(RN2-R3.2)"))
 (segment (start 115.962501 106.775) (end 116.625 106.775) (width 0.2) (layer "F.Cu") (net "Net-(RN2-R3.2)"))
 (segment (start 112.25 116.025) (end 114.675 116.025) (width 0.2) (layer "F.Cu") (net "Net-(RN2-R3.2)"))
 (segment (start 115.6625 104.534448) (end 115.6625 106.474999) (width 0.2) (layer "F.Cu") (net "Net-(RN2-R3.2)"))
 (segment (start 115.412499 116.025) (end 116.625 114.812499) (width 0.2) (layer "F.Cu") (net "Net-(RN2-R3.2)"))
 (segment (start 117.3 97.875) (end 117.3 102.896948) (width 0.2) (layer "F.Cu") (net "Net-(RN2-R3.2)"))
 (segment (start 114.675 116.025) (end 115.412499 116.025) (width 0.2) (layer "F.Cu") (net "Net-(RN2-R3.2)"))
 (segment (start 116.625 114.812499) (end 116.625 106.775) (width 0.2) (layer "F.Cu") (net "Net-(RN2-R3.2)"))
 (segment (start 117.3 102.896948) (end 115.6625 104.534448) (width 0.2) (layer "F.Cu") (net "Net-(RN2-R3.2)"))
 (segment (start 115.6625 106.474999) (end 115.962501 106.775) (width 0.2) (layer "F.Cu") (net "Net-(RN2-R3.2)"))
 (segment (start 123.09 116.025) (end 123.94 116.875) (width 0.2) (layer "F.Cu") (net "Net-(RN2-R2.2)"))
 (segment (start 120.4 116.025) (end 123.09 116.025) (width 0.2) (layer "F.Cu") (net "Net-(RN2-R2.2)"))
 (segment (start 118.5 107.175) (end 118.5 116.075) (width 0.2) (layer "F.Cu") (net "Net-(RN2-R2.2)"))
 (segment (start 117.8 106.775) (end 117.8 98.175) (width 0.2) (layer "F.Cu") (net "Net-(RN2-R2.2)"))
 (segment (start 120.4 116.025) (end 119.7625 116.025) (width 0.2) (layer "F.Cu") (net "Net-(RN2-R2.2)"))
 (segment (start 117.8 98.175) (end 118.1 97.875) (width 0.2) (layer "F.Cu") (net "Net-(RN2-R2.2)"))
 (segment (start 118.9 106.775) (end 118.5 107.175) (width 0.2) (layer "F.Cu") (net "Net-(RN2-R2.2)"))
 (segment (start 118.9 106.775) (end 117.8 106.775) (width 0.2) (layer "F.Cu") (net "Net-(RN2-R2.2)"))
 (segment (start 119.7625 116.025) (end 119.7625 116.075) (width 0.2) (layer "F.Cu") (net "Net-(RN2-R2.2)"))
 (via (at 118.5 116.075) (size 0.6) (drill 0.3) (layers "F.Cu" "B.Cu") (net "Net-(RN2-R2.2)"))
 (segment (start 118.5 116.075) (end 120.3 116.075) (width 0.2) (layer "B.Cu") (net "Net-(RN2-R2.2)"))
 (segment (start 120.5 104.875) (end 120.7 105.075) (width 0.2) (layer "F.Cu") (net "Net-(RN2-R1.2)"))
 (segment (start 120.7 105.075) (end 120.7 109.595) (width 0.2) (layer "F.Cu") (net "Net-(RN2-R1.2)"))
 (segment (start 118.9 97.875) (end 118.9 104.875) (width 0.2) (layer "F.Cu") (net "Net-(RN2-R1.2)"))
 (segment (start 121.55 114.725) (end 123.4 112.875) (width 0.2) (layer "F.Cu") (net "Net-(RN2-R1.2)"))
 (segment (start 118.9 104.875) (end 120.5 104.875) (width 0.2) (layer "F.Cu") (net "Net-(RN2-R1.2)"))
 (segment (start 120.4 114.725) (end 121.55 114.725) (width 0.2) (layer "F.Cu") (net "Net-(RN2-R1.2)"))
 (segment (start 120.7 109.595) (end 123.98 112.875) (width 0.2) (layer "F.Cu") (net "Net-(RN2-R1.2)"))
 (segment (start 123.4 112.875) (end 123.98 112.875) (width 0.2) (layer "F.Cu") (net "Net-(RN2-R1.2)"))
 (segment (start 110.91 99.365) (end 111.89 99.365) (width 0.2) (layer "F.Cu") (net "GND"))
 (segment (start 110.4 99.375) (end 110.9 99.375) (width 0.2) (layer "F.Cu") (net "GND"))
 (segment (start 110.4 103.865) (end 110.4 99.375) (width 0.2) (layer "F.Cu") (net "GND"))
 (segment (start 111.9 105.365) (end 110.4 103.865) (width 0.2) (layer "F.Cu") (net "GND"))
 (segment (start 110.9 99.375) (end 110.91 99.365) (width 0.2) (layer "F.Cu") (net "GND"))
 (segment (start 126.4 102.775) (end 126.4 97.395) (width 0.2) (layer "F.Cu") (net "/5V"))
 (segment (start 123.9 104.875) (end 122.2 104.875) (width 0.2) (layer "F.Cu") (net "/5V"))
 (segment (start 120.4 115.375) (end 124.388067 115.375) (width 0.2) (layer "F.Cu") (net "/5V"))
 (segment (start 124.388067 115.375) (end 126 113.763067) (width 0.2) (layer "F.Cu") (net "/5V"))
 (segment (start 126.4 97.395) (end 124.39 95.385) (width 0.2) (layer "F.Cu") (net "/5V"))
 (segment (start 126 113.763067) (end 126 107.16) (width 0.2) (layer "F.Cu") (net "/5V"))
 (segment (start 126.4 105.19) (end 126.4 102.775) (width 0.2) (layer "F.Cu") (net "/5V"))
 (segment (start 126 107.16) (end 125.215 106.375) (width 0.2) (layer "F.Cu") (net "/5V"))
 (segment (start 124.065 105.14) (end 124.065 104.875) (width 0.2) (layer "F.Cu") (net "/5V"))
 (segment (start 125.215 106.375) (end 126.4 105.19) (width 0.2) (layer "F.Cu") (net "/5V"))
 (segment (start 125.215 106.375) (end 125.215 106.29) (width 0.2) (layer "F.Cu") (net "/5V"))
 (segment (start 125.215 106.29) (end 124.065 105.14) (width 0.2) (layer "F.Cu") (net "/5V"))
 (via (at 122.2 104.875) (size 0.6) (drill 0.3) (layers "F.Cu" "B.Cu") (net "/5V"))
 (segment (start 120.9 105.875) (end 118.9 105.875) (width 0.2) (layer "B.Cu") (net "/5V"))
 (segment (start 122.2 104.875) (end 121.9 104.875) (width 0.2) (layer "B.Cu") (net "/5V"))
 (segment (start 121.9 104.875) (end 120.9 105.875) (width 0.2) (layer "B.Cu") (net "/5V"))
 (segment (start 111.4 121.375) (end 111.4 120.275) (width 0.2) (layer "F.Cu") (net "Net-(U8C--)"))
 (segment (start 111.4 120.275) (end 112.9 118.775) (width 0.2) (layer "F.Cu") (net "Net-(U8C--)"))
 (segment (start 112.9 117.275) (end 113 117.175) (width 0.2) (layer "F.Cu") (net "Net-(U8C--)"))
 (segment (start 112.9 118.775) (end 112.9 117.275) (width 0.2) (layer "F.Cu") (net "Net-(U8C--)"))
 (via (at 113 117.175) (size 0.6) (drill 0.3) (layers "F.Cu" "B.Cu") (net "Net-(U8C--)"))
 (segment (start 113 117.175) (end 113 113.475) (width 0.2) (layer "B.Cu") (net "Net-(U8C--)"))
 (segment (start 114.8 113.475) (end 114.8 114.075) (width 0.2) (layer "B.Cu") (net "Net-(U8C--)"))
 (segment (start 113 113.475) (end 114.8 113.475) (width 0.2) (layer "B.Cu") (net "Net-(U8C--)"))
 (segment (start 120.4 114.075) (end 120.4 113.425) (width 0.2) (layer "F.Cu") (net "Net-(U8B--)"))
 (segment (start 119.662501 114.075) (end 120.4 114.075) (width 0.2) (layer "F.Cu") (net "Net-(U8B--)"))
 (segment (start 119.3625 114.375001) (end 119.662501 114.075) (width 0.2) (layer "F.Cu") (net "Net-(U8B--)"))
 (segment (start 119.3625 120.3375) (end 119.3625 114.375001) (width 0.2) (layer "F.Cu") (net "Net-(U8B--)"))
 (segment (start 120.4 121.375) (end 119.3625 120.3375) (width 0.2) (layer "F.Cu") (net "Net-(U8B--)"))
 (segment (start 120.4 116.675) (end 120.4 117.325) (width 0.2) (layer "F.Cu") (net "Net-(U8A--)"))
 (segment (start 124.4 121.325) (end 120.4 117.325) (width 0.2) (layer "F.Cu") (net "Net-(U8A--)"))
 (segment (start 124.4 121.55) (end 124.4 121.325) (width 0.2) (layer "F.Cu") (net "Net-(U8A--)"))
 (segment (start 115.9 118.55) (end 114.675 117.325) (width 0.2) (layer "F.Cu") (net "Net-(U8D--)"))
 (segment (start 114.675 116.675) (end 114.675 117.325) (width 0.2) (layer "F.Cu") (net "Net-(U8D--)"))
 (segment (start 115.9 121.375) (end 115.9 118.55) (width 0.2) (layer "F.Cu") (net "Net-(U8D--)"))
 (segment (start 120.4 125.375) (end 120.4 123.025) (width 0.2) (layer "F.Cu") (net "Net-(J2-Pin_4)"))
 (segment (start 121.175 125.375) (end 120.4 125.375) (width 0.2) (layer "F.Cu") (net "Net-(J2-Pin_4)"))
 (segment (start 122.1 126.3) (end 121.175 125.375) (width 0.2) (layer "F.Cu") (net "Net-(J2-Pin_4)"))
 (segment (start 126.305 136.835) (end 122.1 132.63) (width 0.2) (layer "F.Cu") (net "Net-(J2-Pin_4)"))
 (segment (start 122.1 132.63) (end 122.1 126.3) (width 0.2) (layer "F.Cu") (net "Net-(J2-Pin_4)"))
 (segment (start 121.225 136.835) (end 123.19 138.8) (width 0.2) (layer "F.Cu") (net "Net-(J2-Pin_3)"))
 (segment (start 124.4 125.375) (end 124.4 123.2) (width 0.2) (layer "F.Cu") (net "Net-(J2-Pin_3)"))
 (segment (start 128.1 125.3) (end 128.025 125.375) (width 0.2) (layer "F.Cu") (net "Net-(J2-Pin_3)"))
 (segment (start 128.5 125.7) (end 128.1 125.3) (width 0.2) (layer "F.Cu") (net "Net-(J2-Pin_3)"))
 (segment (start 128.5 138.8) (end 128.5 125.7) (width 0.2) (layer "F.Cu") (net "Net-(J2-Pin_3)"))
 (segment (start 123.19 138.8) (end 128.5 138.8) (width 0.2) (layer "F.Cu") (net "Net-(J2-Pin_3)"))
 (segment (start 128.025 125.375) (end 124.4 125.375) (width 0.2) (layer "F.Cu") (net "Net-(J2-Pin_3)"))
 (segment (start 117.475 125.375) (end 117.6 125.5) (width 0.2) (layer "F.Cu") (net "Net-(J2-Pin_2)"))
 (segment (start 115.9 125.375) (end 117.475 125.375) (width 0.2) (layer "F.Cu") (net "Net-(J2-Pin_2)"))
 (segment (start 115.9 125.375) (end 115.9 123.025) (width 0.2) (layer "F.Cu") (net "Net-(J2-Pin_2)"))
 (segment (start 117.6 135.38) (end 116.145 136.835) (width 0.2) (layer "F.Cu") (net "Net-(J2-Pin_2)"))
 (segment (start 117.6 125.5) (end 117.6 135.38) (width 0.2) (layer "F.Cu") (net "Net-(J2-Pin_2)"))
 (segment (start 113 125.4) (end 112.975 125.375) (width 0.2) (layer "F.Cu") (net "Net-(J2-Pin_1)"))
 (segment (start 112.975 125.375) (end 111.4 125.375) (width 0.2) (layer "F.Cu") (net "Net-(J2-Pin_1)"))
 (segment (start 113.1 132) (end 113 131.9) (width 0.2) (layer "F.Cu") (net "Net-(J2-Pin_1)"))
 (segment (start 111.065 134.035) (end 113.1 132) (width 0.2) (layer "F.Cu") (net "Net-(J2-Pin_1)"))
 (segment (start 111.065 136.835) (end 111.065 134.035) (width 0.2) (layer "F.Cu") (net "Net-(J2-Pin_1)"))
 (segment (start 113 131.9) (end 113 125.4) (width 0.2) (layer "F.Cu") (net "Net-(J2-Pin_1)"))
 (segment (start 111.4 125.375) (end 111.4 123.025) (width 0.2) (layer "F.Cu") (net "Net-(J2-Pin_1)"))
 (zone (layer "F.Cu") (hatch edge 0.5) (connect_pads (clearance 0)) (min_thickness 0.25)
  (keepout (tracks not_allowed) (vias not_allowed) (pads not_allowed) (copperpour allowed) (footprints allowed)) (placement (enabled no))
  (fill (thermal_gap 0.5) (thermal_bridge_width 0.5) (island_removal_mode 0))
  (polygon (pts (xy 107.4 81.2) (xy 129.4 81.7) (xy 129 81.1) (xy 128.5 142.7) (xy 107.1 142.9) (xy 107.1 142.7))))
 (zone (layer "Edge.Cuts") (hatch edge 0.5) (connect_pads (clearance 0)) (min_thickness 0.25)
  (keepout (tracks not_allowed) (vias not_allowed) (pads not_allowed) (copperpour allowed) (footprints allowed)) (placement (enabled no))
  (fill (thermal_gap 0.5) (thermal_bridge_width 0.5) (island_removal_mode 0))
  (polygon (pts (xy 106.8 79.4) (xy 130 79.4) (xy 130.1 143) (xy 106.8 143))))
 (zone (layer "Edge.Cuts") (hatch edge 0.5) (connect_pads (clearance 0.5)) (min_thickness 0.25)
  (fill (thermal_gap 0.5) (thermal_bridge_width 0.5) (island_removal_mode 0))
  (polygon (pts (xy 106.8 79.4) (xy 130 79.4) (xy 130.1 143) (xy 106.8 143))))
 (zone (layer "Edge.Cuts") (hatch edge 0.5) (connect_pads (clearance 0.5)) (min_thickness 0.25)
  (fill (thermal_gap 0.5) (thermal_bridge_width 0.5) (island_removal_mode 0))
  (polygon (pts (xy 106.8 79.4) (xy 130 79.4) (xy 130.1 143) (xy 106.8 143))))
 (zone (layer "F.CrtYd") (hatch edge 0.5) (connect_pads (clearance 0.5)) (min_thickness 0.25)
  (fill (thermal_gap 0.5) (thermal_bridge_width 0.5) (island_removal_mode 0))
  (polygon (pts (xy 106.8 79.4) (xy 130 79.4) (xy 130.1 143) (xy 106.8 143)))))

